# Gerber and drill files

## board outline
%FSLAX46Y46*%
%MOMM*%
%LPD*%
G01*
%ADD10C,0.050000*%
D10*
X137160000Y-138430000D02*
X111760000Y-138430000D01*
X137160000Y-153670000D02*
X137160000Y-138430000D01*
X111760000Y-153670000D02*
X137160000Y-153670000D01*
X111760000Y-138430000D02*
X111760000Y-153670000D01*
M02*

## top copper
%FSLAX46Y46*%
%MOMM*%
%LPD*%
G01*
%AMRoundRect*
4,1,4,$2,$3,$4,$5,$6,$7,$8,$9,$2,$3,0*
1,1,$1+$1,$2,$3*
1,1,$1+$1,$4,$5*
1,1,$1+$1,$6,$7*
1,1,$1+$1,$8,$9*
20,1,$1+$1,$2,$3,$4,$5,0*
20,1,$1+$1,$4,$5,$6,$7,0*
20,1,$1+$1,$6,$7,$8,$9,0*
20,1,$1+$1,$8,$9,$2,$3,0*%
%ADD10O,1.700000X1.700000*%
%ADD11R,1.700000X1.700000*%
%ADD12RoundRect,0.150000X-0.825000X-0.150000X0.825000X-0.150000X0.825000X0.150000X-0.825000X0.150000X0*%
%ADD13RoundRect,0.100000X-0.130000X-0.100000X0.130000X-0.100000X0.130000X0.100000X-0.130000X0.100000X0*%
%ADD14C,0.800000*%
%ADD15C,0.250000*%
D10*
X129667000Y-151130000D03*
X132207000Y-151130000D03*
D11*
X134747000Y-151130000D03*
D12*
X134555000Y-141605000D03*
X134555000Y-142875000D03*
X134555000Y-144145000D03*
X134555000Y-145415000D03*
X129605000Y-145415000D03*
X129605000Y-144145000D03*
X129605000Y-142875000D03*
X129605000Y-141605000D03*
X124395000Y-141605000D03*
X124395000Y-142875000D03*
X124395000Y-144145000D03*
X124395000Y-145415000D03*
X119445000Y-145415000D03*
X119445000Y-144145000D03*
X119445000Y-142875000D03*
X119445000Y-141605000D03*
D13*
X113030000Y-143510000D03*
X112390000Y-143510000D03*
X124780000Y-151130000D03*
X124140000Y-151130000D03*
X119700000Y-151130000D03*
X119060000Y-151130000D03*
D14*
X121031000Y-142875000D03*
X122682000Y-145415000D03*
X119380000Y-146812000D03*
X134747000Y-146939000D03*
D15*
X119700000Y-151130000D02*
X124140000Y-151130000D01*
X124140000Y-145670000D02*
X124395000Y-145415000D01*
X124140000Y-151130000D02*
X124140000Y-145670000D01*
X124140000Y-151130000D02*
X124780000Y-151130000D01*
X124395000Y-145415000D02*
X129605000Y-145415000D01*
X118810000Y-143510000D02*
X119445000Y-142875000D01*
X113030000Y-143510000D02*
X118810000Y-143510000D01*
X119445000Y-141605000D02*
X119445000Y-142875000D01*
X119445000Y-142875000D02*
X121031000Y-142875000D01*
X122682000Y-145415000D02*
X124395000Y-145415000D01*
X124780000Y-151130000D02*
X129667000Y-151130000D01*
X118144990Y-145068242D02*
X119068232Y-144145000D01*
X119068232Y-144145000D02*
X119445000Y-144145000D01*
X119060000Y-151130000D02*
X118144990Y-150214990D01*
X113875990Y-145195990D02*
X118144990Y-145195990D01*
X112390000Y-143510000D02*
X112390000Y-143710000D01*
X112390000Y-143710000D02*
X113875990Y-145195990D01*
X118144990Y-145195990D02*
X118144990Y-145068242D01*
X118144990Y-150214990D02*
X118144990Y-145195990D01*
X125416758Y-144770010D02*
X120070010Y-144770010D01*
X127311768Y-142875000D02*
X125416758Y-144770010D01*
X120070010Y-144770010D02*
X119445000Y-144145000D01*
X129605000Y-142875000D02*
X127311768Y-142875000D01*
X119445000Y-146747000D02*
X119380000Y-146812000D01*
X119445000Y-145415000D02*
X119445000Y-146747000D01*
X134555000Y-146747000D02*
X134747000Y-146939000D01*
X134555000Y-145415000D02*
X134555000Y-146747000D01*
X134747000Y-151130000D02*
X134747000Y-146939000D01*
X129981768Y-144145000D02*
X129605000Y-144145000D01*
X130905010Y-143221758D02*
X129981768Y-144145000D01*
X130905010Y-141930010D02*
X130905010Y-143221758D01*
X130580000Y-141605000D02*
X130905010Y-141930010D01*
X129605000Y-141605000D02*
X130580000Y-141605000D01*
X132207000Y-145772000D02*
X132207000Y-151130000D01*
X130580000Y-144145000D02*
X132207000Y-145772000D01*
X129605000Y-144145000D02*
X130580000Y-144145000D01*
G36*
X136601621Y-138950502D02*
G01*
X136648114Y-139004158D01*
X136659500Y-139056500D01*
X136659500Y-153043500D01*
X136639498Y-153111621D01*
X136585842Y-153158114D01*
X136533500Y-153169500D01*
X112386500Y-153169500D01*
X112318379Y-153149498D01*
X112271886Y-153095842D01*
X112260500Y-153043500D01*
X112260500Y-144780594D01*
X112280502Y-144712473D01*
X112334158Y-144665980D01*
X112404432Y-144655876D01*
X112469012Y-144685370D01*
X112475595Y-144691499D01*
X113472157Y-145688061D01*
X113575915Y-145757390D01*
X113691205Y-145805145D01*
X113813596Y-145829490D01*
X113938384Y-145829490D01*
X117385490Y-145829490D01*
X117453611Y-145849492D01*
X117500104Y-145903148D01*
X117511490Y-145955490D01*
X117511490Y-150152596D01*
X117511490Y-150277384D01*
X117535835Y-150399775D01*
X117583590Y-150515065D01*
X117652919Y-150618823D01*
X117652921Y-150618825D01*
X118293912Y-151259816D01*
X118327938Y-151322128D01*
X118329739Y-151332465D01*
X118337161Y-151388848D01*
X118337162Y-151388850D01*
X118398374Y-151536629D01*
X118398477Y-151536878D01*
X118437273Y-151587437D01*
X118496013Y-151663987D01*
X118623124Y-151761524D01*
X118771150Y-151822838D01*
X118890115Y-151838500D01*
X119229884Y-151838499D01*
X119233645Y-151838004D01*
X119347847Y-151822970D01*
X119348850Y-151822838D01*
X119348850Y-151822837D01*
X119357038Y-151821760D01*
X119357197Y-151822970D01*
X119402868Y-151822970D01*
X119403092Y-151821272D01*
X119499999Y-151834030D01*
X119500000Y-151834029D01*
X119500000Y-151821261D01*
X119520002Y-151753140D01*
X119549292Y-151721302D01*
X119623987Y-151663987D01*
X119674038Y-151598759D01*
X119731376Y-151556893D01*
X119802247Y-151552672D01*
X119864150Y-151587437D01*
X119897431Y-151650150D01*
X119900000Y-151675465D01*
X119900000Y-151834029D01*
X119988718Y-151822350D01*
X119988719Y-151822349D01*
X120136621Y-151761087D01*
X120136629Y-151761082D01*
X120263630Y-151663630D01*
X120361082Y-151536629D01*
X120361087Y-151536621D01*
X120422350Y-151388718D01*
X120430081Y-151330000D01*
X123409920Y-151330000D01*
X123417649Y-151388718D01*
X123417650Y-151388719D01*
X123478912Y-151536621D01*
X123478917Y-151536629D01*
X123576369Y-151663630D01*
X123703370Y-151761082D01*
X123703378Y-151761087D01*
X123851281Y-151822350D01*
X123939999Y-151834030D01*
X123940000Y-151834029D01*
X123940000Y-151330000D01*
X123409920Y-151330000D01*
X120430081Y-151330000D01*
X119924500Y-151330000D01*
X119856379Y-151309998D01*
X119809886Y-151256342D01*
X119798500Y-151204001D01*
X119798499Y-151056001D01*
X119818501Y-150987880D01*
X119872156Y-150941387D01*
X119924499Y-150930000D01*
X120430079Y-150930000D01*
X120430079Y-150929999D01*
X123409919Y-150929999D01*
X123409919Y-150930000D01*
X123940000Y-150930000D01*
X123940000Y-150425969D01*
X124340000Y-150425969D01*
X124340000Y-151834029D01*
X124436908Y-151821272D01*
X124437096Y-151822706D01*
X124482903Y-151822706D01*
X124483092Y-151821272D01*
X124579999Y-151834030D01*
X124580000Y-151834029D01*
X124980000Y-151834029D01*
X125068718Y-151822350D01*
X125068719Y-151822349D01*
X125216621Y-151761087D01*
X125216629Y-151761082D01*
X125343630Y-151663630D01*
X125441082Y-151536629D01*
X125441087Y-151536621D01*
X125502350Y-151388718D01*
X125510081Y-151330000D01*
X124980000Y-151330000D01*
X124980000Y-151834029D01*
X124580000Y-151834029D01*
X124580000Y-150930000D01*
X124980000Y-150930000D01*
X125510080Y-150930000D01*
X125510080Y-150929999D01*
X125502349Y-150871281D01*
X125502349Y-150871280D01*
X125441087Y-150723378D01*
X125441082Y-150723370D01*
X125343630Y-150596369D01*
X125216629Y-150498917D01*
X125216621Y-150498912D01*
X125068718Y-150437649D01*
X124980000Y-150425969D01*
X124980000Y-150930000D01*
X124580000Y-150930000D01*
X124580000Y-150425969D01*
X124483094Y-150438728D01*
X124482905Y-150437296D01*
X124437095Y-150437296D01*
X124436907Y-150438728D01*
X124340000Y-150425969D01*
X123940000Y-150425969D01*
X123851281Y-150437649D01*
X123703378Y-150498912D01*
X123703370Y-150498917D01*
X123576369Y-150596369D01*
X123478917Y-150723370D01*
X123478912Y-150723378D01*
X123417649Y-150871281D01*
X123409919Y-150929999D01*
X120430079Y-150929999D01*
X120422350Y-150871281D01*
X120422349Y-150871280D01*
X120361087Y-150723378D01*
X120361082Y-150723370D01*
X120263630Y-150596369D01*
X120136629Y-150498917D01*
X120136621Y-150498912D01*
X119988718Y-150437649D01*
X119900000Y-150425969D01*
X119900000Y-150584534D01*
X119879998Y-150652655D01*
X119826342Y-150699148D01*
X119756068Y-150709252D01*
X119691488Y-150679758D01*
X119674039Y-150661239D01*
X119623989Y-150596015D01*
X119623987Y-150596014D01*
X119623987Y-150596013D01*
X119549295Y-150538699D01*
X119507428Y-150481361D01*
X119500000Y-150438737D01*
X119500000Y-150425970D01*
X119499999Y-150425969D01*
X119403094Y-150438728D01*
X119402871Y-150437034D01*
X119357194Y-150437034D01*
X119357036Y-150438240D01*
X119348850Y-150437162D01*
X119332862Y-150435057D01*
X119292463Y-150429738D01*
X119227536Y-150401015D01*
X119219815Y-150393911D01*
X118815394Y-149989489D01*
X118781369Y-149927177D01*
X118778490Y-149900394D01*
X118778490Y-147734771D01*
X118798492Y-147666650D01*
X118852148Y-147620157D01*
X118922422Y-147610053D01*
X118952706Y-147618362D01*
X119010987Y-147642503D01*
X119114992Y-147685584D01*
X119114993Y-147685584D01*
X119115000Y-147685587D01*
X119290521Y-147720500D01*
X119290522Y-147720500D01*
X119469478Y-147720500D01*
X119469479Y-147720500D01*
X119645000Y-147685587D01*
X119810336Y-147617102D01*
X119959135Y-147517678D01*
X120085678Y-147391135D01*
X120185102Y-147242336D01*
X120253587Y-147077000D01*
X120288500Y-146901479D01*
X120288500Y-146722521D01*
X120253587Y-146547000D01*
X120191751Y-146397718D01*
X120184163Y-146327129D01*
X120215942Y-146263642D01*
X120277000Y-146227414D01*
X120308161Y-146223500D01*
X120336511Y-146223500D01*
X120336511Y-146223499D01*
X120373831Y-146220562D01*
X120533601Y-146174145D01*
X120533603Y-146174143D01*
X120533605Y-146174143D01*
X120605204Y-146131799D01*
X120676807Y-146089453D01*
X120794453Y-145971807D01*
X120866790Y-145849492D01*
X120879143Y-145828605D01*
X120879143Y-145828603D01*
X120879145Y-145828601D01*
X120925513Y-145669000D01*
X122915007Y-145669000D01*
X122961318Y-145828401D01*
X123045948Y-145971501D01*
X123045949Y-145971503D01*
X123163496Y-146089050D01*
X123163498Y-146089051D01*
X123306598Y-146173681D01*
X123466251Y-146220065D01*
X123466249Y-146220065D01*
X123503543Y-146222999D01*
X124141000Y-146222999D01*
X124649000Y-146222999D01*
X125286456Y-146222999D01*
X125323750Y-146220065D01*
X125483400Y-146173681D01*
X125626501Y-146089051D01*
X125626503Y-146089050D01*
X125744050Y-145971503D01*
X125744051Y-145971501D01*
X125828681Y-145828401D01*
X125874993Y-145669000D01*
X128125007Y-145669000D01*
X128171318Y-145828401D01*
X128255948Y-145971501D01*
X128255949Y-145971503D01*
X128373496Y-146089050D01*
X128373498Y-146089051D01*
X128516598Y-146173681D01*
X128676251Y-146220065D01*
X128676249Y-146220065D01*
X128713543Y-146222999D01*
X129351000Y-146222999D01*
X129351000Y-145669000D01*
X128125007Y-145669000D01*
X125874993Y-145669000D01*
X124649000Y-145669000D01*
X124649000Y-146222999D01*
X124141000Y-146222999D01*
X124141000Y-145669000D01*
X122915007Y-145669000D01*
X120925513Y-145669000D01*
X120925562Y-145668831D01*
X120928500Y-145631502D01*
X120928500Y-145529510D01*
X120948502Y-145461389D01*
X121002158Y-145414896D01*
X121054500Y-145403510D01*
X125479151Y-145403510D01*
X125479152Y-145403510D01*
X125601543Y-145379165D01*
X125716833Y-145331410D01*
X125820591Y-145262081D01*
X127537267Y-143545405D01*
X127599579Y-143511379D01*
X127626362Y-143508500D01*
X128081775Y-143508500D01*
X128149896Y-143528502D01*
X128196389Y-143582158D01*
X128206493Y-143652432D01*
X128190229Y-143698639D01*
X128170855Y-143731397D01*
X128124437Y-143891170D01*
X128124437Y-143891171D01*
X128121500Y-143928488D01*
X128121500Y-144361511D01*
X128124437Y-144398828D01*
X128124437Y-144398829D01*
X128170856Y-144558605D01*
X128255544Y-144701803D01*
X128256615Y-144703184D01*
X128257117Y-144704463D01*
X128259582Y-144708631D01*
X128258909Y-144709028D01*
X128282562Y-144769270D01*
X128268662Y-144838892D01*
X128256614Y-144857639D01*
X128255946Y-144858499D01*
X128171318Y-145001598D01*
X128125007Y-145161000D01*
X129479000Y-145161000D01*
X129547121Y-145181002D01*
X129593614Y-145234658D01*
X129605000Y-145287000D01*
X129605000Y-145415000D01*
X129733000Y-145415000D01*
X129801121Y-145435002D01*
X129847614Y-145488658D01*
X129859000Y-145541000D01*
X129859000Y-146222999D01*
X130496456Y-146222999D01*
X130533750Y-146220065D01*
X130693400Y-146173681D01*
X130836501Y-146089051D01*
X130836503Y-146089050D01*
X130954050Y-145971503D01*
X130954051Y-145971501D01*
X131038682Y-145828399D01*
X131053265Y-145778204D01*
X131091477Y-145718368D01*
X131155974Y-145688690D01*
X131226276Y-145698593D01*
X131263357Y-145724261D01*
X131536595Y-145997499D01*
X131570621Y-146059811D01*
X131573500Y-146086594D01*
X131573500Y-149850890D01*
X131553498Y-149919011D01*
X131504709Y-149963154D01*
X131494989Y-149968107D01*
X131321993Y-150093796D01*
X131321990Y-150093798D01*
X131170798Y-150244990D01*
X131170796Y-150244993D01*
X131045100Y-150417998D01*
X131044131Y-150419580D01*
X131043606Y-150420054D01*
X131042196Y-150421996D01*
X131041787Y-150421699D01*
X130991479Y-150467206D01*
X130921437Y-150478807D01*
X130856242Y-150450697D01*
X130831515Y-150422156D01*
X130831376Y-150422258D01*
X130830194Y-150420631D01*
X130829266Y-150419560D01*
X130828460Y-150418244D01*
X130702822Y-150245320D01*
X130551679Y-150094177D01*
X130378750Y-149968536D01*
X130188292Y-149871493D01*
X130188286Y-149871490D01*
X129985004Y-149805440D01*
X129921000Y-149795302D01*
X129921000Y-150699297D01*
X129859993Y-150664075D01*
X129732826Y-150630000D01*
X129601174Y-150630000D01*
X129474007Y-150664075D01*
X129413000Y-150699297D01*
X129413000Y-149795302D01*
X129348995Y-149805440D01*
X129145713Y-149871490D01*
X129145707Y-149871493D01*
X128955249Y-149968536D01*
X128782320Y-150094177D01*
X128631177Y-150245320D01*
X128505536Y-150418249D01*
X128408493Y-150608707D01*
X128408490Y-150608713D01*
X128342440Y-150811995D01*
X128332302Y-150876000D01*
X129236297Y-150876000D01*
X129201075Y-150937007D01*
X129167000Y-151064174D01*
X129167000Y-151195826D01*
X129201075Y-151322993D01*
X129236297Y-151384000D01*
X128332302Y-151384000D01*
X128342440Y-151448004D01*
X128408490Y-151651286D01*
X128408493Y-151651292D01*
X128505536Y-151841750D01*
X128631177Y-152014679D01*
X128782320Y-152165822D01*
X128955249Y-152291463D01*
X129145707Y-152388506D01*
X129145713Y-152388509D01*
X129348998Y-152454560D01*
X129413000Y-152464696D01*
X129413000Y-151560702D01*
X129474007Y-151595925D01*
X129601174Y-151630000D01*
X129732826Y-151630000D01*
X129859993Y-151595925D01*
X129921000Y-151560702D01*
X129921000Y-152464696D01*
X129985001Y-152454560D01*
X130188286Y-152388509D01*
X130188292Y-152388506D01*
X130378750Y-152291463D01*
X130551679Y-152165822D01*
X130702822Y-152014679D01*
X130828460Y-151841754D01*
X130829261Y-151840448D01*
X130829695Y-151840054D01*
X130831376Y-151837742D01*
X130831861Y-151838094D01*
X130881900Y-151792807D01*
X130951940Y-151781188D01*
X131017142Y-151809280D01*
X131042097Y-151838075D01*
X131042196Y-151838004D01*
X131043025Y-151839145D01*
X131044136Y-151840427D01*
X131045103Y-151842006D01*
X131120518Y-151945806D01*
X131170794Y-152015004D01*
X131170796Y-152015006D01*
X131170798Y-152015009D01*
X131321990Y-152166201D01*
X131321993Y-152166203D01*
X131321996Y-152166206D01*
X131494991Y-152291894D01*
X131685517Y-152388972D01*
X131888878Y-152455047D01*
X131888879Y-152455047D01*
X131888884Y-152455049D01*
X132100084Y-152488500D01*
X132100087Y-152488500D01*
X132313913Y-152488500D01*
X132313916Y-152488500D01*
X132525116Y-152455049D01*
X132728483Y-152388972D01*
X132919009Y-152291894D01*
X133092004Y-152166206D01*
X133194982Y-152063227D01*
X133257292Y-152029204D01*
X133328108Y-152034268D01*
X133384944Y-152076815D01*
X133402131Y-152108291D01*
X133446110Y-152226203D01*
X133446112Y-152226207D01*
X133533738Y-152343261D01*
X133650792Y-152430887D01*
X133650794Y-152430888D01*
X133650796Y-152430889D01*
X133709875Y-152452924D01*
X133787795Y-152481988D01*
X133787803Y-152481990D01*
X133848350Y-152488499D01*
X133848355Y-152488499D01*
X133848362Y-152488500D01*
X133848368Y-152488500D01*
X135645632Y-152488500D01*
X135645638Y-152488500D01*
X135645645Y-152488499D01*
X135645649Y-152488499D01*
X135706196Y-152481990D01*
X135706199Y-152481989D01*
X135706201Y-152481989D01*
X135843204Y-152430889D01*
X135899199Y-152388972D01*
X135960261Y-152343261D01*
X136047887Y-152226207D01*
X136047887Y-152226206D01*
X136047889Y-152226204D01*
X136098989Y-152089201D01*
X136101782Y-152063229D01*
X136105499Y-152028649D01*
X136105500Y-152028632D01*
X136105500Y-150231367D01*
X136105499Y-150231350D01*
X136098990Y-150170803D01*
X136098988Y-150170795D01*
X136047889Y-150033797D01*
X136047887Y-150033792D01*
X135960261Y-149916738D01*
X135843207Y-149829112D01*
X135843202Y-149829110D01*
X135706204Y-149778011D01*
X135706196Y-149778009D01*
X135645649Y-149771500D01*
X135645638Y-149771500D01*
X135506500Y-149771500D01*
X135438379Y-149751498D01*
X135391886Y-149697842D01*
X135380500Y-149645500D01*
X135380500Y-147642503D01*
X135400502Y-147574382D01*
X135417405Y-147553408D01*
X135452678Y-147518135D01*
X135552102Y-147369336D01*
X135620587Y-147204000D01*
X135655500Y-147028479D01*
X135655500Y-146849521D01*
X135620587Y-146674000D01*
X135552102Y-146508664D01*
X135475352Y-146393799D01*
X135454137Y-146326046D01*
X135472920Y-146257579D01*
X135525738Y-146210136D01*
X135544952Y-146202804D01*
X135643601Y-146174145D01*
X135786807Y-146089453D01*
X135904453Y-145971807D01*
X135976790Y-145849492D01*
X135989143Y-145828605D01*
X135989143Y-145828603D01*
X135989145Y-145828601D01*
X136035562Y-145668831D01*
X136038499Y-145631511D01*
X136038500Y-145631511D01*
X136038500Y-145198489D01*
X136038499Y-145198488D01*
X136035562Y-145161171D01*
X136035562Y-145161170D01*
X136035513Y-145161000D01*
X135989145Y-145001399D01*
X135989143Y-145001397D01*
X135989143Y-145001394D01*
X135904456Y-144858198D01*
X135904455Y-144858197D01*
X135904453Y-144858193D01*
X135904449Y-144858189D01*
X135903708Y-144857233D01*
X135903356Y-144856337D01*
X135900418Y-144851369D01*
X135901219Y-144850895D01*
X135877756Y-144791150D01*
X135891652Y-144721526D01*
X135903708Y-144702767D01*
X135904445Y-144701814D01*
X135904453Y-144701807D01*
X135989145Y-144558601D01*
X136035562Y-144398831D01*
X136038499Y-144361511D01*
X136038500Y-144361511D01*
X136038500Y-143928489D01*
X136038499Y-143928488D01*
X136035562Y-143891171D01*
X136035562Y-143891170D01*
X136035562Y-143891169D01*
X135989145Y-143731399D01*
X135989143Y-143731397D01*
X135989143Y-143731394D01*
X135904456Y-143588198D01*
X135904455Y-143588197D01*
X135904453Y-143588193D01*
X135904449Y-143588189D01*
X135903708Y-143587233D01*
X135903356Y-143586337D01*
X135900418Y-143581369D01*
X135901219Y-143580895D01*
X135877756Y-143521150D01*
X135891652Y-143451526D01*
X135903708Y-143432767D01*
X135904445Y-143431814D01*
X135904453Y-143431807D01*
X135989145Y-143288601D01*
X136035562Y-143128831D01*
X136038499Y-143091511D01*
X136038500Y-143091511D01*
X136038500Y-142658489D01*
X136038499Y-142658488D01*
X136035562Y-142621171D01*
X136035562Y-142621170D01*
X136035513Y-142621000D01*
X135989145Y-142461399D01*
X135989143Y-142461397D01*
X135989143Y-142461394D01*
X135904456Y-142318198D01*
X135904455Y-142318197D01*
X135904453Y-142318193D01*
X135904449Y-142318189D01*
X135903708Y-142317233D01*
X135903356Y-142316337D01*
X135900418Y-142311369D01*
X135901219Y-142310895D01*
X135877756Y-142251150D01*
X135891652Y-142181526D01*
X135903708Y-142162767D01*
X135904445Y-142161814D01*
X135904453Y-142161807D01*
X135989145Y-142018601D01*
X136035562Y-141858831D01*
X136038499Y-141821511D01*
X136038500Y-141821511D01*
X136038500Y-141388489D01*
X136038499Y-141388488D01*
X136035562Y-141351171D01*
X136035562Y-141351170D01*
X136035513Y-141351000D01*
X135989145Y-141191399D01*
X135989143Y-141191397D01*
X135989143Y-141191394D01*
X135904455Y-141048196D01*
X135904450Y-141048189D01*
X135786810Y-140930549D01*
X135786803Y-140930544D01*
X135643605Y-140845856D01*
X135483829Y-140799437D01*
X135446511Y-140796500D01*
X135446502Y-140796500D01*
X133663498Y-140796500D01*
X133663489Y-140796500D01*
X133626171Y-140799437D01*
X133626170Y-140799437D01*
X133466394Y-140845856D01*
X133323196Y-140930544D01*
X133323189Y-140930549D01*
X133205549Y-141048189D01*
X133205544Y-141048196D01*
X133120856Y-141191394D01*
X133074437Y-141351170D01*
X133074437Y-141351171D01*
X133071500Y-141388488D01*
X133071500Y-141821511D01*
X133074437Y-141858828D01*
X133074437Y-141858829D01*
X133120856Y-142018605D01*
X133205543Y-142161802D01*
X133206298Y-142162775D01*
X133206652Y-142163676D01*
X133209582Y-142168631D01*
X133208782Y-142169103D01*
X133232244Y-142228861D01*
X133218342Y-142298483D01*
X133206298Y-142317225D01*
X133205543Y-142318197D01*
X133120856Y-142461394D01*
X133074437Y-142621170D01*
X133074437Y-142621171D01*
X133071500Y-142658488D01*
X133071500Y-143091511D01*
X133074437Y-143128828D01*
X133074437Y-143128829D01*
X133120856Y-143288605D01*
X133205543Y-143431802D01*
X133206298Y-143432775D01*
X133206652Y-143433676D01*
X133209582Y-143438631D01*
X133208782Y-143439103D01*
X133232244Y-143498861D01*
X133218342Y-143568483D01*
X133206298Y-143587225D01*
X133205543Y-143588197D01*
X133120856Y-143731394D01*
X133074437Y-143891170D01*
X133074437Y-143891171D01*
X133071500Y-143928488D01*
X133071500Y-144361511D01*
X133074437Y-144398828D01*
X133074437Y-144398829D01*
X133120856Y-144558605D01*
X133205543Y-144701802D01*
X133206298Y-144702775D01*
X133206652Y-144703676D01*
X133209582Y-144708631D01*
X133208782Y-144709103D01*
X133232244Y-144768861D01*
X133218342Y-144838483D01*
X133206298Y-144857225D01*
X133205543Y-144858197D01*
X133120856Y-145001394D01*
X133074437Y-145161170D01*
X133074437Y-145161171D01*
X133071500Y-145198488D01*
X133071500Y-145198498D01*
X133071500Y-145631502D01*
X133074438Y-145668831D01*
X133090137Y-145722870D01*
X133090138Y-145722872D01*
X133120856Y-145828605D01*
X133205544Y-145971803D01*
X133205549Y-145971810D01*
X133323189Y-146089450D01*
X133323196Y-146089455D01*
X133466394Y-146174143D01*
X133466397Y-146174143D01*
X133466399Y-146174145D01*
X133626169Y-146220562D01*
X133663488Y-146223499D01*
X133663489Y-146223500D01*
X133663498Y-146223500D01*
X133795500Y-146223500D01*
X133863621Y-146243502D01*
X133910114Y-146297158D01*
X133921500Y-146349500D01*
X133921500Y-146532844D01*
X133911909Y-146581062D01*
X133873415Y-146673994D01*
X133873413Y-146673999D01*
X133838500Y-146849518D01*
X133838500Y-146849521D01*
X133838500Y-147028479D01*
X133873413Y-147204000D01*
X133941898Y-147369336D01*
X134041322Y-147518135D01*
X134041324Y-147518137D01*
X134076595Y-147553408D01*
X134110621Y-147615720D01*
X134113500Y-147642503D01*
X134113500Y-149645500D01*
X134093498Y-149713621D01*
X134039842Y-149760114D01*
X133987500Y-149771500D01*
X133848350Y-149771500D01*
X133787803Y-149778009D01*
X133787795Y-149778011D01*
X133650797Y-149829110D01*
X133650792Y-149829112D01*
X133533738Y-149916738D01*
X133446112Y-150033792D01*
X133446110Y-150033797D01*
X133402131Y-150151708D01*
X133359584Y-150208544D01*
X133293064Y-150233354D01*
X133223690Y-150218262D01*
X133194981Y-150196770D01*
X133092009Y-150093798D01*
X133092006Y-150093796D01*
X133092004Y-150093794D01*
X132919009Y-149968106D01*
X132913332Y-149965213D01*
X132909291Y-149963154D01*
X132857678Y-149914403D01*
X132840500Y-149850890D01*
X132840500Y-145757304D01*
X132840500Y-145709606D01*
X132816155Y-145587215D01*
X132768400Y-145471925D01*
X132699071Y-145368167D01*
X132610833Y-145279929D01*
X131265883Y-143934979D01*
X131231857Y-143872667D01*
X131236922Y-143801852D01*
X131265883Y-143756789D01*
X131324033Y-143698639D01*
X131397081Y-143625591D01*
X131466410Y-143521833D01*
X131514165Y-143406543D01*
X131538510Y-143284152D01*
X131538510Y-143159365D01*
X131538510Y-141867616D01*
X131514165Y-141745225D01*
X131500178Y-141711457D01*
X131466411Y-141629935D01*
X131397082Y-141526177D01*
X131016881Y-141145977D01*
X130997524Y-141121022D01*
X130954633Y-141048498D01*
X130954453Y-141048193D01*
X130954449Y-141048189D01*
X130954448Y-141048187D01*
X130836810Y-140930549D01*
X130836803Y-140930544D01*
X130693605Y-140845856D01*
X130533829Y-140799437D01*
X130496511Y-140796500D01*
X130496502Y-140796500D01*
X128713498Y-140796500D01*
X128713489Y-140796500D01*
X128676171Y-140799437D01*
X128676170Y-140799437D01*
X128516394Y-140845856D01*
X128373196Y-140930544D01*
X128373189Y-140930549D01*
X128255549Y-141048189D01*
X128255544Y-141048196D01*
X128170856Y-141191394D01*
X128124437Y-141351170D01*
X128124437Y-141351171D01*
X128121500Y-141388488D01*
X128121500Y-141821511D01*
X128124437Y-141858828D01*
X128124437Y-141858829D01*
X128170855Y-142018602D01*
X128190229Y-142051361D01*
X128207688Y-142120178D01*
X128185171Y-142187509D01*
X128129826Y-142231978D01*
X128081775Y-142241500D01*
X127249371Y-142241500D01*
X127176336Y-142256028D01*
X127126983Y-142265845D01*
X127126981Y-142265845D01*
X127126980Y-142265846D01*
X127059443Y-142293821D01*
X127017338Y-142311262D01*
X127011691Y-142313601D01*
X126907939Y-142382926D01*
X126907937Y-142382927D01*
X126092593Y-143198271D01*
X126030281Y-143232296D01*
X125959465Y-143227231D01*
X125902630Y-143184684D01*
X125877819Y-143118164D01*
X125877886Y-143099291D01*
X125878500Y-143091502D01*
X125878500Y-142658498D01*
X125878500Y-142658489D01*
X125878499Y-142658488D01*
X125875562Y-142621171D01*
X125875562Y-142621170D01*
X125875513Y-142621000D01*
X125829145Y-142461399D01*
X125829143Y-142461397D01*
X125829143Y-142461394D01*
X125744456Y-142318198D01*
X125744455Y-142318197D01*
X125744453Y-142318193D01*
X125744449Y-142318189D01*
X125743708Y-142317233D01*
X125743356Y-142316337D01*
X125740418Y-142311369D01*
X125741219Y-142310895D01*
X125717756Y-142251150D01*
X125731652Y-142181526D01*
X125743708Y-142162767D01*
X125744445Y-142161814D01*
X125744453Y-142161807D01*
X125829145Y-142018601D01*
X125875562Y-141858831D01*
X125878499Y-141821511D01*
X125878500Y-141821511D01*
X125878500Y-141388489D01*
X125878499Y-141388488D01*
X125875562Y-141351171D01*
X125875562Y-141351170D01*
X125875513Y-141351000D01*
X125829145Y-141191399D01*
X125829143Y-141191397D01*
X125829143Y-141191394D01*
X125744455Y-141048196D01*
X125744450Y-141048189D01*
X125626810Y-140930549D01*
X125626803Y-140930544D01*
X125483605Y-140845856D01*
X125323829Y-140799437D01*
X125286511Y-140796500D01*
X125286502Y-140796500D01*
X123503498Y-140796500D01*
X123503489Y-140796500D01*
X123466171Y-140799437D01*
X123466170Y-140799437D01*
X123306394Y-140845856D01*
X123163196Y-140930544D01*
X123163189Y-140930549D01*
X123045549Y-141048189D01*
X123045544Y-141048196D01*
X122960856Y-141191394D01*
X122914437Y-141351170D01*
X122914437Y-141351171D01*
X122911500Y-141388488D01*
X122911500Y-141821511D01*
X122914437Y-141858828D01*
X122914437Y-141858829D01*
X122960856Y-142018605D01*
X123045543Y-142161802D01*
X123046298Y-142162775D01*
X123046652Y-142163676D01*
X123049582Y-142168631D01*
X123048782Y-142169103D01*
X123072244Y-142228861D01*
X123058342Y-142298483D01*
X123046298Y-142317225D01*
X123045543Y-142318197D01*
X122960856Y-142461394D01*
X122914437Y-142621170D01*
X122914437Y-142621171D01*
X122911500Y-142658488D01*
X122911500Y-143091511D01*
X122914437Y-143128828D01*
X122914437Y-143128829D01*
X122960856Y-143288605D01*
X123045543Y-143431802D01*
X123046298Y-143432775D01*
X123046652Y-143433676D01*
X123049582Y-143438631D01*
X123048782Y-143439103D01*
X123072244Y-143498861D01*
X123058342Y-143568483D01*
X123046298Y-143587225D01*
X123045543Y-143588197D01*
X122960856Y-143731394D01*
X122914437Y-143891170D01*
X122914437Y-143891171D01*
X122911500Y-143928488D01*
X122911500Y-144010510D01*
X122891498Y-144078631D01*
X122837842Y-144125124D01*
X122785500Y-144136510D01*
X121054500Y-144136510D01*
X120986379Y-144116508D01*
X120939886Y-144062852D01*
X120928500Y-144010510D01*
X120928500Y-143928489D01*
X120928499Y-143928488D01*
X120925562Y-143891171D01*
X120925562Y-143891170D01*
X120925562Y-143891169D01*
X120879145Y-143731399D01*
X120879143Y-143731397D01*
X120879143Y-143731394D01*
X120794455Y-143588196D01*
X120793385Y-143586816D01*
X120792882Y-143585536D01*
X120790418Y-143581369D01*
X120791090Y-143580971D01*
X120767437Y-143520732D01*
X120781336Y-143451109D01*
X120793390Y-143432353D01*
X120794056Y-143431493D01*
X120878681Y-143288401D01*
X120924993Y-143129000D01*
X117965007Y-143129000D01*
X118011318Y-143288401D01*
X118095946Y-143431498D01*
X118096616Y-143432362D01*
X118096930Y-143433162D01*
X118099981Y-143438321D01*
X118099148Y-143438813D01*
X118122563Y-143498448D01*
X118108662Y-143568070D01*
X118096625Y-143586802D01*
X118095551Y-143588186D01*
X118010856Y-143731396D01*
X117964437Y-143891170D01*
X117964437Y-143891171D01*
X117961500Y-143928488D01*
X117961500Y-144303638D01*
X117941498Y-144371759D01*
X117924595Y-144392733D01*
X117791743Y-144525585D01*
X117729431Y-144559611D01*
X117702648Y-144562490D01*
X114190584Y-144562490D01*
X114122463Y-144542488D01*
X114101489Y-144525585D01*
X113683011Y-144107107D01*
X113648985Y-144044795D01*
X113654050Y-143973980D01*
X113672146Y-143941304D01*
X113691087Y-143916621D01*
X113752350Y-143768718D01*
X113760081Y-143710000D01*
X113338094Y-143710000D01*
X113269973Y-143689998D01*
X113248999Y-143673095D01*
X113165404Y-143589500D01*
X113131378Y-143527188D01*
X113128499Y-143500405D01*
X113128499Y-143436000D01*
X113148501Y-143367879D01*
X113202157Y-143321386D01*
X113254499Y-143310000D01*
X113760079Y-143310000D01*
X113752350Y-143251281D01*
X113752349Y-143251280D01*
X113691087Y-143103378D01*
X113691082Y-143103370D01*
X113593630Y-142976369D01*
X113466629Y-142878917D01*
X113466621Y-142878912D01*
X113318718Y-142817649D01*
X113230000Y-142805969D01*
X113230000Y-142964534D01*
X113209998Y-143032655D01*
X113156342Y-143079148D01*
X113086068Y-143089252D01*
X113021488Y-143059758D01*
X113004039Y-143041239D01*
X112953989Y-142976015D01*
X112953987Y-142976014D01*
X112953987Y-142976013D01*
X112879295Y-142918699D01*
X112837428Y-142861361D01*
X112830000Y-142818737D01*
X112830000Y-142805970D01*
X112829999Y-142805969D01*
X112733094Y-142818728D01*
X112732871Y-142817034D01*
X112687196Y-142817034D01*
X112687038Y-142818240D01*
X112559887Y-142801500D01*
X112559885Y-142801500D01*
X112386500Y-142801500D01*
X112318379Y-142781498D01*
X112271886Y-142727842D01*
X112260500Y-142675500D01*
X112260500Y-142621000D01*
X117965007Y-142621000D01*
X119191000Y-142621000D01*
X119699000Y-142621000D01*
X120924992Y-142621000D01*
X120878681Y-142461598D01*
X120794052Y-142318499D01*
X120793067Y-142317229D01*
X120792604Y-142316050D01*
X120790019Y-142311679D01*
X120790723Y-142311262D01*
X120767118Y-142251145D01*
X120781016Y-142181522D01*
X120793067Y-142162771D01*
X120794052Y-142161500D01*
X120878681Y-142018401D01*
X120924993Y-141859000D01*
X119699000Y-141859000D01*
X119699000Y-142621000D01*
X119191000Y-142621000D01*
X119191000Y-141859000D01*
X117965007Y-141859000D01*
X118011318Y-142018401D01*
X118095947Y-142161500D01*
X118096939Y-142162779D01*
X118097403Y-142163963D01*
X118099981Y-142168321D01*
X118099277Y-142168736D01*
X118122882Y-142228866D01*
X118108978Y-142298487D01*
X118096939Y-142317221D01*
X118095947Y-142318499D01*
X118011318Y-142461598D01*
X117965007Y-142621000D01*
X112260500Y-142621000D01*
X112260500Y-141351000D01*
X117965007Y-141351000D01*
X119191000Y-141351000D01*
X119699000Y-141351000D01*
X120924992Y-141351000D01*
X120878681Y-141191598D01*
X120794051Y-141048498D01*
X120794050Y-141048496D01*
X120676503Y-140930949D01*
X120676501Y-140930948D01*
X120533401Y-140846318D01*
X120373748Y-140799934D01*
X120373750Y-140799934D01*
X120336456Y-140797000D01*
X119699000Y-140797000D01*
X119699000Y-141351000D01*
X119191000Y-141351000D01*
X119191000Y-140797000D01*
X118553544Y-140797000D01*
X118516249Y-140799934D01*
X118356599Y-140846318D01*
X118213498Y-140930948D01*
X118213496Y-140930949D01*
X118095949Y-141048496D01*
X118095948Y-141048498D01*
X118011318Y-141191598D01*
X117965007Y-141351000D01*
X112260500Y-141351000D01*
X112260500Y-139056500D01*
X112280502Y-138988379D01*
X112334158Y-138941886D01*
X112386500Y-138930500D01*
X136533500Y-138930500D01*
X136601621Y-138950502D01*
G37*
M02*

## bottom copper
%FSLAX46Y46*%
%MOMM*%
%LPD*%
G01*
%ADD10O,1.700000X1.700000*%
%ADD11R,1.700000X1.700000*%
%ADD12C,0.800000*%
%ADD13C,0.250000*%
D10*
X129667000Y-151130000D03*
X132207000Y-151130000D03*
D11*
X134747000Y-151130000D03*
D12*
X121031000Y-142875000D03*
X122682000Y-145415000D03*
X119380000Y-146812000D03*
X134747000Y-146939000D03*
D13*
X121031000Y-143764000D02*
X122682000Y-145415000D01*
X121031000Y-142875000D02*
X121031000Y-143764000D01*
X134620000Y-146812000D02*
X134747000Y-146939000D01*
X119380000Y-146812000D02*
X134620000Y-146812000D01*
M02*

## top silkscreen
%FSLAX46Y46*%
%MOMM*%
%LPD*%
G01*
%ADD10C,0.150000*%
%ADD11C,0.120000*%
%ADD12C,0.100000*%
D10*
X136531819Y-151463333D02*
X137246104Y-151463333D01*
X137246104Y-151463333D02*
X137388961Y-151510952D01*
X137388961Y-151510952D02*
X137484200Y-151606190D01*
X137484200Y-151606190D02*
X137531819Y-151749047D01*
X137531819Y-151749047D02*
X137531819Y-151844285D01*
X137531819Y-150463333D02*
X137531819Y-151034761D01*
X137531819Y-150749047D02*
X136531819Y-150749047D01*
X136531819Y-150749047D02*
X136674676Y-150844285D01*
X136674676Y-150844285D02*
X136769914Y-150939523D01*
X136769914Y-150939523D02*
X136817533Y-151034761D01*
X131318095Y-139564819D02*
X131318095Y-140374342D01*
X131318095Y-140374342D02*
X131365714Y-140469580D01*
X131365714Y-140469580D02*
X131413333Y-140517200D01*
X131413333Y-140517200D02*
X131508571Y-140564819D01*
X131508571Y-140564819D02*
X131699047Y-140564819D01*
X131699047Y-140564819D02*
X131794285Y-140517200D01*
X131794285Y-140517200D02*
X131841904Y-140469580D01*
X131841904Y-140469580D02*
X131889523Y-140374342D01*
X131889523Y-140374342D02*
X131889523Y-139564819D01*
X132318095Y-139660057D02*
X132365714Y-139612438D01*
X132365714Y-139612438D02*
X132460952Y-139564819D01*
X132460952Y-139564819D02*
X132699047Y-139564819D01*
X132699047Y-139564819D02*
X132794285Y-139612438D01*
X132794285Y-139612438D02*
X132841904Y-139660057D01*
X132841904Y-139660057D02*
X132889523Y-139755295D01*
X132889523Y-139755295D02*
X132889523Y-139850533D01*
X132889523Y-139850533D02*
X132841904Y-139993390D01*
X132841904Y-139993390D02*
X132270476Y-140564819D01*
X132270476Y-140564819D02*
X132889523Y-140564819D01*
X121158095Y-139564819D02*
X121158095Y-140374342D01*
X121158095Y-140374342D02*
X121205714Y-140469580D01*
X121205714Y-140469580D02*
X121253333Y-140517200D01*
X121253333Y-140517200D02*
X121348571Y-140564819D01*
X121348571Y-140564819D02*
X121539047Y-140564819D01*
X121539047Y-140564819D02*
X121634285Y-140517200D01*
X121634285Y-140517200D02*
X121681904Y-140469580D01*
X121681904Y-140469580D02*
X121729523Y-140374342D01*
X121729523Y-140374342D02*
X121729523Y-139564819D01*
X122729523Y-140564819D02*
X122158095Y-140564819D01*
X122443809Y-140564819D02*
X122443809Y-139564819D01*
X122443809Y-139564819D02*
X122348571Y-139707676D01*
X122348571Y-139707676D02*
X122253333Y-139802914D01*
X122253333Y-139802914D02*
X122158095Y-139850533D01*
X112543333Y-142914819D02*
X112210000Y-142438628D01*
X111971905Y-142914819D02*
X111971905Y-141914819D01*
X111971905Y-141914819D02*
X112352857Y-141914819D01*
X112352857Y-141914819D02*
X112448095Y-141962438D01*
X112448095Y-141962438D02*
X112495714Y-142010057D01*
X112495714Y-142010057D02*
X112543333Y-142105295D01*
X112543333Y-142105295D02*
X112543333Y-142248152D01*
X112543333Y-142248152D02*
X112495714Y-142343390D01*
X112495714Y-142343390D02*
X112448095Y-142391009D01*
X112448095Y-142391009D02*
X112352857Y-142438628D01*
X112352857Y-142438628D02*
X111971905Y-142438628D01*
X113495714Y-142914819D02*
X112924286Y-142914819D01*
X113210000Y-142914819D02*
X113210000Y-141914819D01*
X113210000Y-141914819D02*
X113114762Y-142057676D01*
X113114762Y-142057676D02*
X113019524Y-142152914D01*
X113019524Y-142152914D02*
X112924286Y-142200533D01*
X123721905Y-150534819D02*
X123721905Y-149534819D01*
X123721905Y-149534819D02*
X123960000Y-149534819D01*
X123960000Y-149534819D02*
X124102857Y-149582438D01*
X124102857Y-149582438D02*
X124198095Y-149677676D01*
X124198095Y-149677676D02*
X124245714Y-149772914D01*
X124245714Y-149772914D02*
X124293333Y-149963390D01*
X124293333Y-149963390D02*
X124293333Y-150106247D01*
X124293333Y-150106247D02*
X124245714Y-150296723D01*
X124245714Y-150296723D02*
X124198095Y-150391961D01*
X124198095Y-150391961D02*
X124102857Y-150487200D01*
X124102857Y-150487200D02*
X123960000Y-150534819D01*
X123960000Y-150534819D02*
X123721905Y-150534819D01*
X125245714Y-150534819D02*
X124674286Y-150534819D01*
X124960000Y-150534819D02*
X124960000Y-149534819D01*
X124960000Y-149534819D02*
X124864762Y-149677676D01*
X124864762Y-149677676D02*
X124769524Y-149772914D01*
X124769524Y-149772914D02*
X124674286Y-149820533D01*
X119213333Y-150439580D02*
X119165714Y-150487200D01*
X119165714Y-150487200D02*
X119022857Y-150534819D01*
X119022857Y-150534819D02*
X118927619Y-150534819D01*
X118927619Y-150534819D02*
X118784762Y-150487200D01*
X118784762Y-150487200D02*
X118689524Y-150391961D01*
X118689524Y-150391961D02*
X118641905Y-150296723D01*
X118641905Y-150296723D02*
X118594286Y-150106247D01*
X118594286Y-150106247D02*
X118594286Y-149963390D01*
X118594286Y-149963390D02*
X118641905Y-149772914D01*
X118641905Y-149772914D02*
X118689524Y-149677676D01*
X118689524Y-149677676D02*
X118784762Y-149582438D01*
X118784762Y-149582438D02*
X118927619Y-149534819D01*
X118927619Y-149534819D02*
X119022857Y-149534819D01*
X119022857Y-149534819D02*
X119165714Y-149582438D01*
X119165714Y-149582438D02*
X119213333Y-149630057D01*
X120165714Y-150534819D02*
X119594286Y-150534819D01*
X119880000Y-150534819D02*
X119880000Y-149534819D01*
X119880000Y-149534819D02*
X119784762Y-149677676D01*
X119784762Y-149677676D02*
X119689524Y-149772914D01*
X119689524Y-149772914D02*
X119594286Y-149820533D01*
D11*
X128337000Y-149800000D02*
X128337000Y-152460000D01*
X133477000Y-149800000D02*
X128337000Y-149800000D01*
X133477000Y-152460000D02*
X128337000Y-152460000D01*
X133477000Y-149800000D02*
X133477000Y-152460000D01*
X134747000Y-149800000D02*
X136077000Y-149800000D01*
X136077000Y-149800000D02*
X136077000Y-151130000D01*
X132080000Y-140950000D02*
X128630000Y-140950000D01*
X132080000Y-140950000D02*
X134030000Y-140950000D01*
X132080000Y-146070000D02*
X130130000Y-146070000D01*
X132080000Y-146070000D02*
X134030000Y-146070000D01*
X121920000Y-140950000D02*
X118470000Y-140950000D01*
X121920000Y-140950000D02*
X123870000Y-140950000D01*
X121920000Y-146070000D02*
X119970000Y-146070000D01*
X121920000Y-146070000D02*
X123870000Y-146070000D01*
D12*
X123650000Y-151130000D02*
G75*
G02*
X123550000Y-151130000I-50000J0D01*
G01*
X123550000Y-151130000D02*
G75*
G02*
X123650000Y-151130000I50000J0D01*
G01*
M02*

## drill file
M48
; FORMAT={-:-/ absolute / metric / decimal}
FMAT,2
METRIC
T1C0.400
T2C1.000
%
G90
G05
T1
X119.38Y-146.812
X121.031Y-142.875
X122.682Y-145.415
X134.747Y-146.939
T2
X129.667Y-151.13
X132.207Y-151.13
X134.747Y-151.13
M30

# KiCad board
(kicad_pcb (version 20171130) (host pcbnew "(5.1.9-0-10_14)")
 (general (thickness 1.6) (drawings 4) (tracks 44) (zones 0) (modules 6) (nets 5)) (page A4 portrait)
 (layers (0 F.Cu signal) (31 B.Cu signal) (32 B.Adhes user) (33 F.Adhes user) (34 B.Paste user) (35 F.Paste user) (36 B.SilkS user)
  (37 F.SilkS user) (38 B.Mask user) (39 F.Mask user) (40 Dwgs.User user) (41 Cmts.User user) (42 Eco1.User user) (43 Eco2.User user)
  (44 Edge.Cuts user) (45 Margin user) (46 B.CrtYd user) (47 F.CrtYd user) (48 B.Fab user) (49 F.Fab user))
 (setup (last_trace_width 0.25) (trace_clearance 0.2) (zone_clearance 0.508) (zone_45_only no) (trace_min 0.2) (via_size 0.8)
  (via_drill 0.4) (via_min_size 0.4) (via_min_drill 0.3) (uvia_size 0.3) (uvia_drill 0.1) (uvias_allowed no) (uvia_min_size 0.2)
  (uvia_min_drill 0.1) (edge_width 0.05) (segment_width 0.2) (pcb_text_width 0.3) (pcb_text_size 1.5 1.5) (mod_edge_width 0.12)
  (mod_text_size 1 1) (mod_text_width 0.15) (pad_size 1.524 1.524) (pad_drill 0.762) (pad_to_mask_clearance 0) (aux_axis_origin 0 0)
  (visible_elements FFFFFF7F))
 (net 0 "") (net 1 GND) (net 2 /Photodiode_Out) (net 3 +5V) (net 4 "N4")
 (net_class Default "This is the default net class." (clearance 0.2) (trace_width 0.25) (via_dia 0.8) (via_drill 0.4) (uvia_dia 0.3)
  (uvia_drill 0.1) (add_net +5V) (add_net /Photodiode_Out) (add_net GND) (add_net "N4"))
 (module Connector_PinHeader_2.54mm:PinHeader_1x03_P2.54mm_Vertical (layer F.Cu) (at 134.747 151.13 270)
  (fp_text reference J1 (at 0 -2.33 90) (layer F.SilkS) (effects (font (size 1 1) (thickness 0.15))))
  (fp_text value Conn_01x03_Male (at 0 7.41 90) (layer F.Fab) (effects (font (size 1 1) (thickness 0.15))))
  (fp_line (start -1.33 6.41) (end 1.33 6.41) (layer F.SilkS) (width 0.12))
  (fp_line (start -1.33 1.27) (end -1.33 6.41) (layer F.SilkS) (width 0.12))
  (fp_line (start 1.33 1.27) (end 1.33 6.41) (layer F.SilkS) (width 0.12))
  (fp_line (start -1.33 1.27) (end 1.33 1.27) (layer F.SilkS) (width 0.12))
  (fp_line (start -1.33 0) (end -1.33 -1.33) (layer F.SilkS) (width 0.12))
  (fp_line (start -1.33 -1.33) (end 0 -1.33) (layer F.SilkS) (width 0.12))
  (pad 3 thru_hole oval (at 0 5.08 270) (size 1.7 1.7) (drill 1) (layers *.Cu *.Mask) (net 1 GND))
  (pad 2 thru_hole oval (at 0 2.54 270) (size 1.7 1.7) (drill 1) (layers *.Cu *.Mask) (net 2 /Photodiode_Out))
  (pad 1 thru_hole rect (at 0 0 270) (size 1.7 1.7) (drill 1) (layers *.Cu *.Mask) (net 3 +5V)))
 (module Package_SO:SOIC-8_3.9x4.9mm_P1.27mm (layer F.Cu) (at 132.08 143.51)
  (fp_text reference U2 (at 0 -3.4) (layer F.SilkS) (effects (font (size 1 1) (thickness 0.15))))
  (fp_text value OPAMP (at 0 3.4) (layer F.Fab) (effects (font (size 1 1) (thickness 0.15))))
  (fp_line (start 0 -2.56) (end -3.45 -2.56) (layer F.SilkS) (width 0.12))
  (fp_line (start 0 -2.56) (end 1.95 -2.56) (layer F.SilkS) (width 0.12))
  (fp_line (start 0 2.56) (end -1.95 2.56) (layer F.SilkS) (width 0.12))
  (fp_line (start 0 2.56) (end 1.95 2.56) (layer F.SilkS) (width 0.12))
  (pad 8 smd roundrect (at 2.475 -1.905) (size 1.95 0.6) (layers F.Cu F.Paste F.Mask) (roundrect_rratio 0.25))
  (pad 7 smd roundrect (at 2.475 -0.635) (size 1.95 0.6) (layers F.Cu F.Paste F.Mask) (roundrect_rratio 0.25))
  (pad 6 smd roundrect (at 2.475 0.635) (size 1.95 0.6) (layers F.Cu F.Paste F.Mask) (roundrect_rratio 0.25))
  (pad 5 smd roundrect (at 2.475 1.905) (size 1.95 0.6) (layers F.Cu F.Paste F.Mask) (roundrect_rratio 0.25) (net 3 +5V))
  (pad 4 smd roundrect (at -2.475 1.905) (size 1.95 0.6) (layers F.Cu F.Paste F.Mask) (roundrect_rratio 0.25) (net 1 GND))
  (pad 3 smd roundrect (at -2.475 0.635) (size 1.95 0.6) (layers F.Cu F.Paste F.Mask) (roundrect_rratio 0.25) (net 2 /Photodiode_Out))
  (pad 2 smd roundrect (at -2.475 -0.635) (size 1.95 0.6) (layers F.Cu F.Paste F.Mask) (roundrect_rratio 0.25) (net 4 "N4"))
  (pad 1 smd roundrect (at -2.475 -1.905) (size 1.95 0.6) (layers F.Cu F.Paste F.Mask) (roundrect_rratio 0.25) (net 2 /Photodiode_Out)))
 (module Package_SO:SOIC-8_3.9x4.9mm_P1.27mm (layer F.Cu) (at 121.92 143.51)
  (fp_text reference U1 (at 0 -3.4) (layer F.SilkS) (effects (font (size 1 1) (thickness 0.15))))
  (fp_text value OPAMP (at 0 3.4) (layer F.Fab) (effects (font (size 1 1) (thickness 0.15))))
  (fp_line (start 0 -2.56) (end -3.45 -2.56) (layer F.SilkS) (width 0.12))
  (fp_line (start 0 -2.56) (end 1.95 -2.56) (layer F.SilkS) (width 0.12))
  (fp_line (start 0 2.56) (end -1.95 2.56) (layer F.SilkS) (width 0.12))
  (fp_line (start 0 2.56) (end 1.95 2.56) (layer F.SilkS) (width 0.12))
  (pad 8 smd roundrect (at 2.475 -1.905) (size 1.95 0.6) (layers F.Cu F.Paste F.Mask) (roundrect_rratio 0.25))
  (pad 7 smd roundrect (at 2.475 -0.635) (size 1.95 0.6) (layers F.Cu F.Paste F.Mask) (roundrect_rratio 0.25))
  (pad 6 smd roundrect (at 2.475 0.635) (size 1.95 0.6) (layers F.Cu F.Paste F.Mask) (roundrect_rratio 0.25))
  (pad 5 smd roundrect (at 2.475 1.905) (size 1.95 0.6) (layers F.Cu F.Paste F.Mask) (roundrect_rratio 0.25) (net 1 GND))
  (pad 4 smd roundrect (at -2.475 1.905) (size 1.95 0.6) (layers F.Cu F.Paste F.Mask) (roundrect_rratio 0.25) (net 3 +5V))
  (pad 3 smd roundrect (at -2.475 0.635) (size 1.95 0.6) (layers F.Cu F.Paste F.Mask) (roundrect_rratio 0.25) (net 4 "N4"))
  (pad 2 smd roundrect (at -2.475 -0.635) (size 1.95 0.6) (layers F.Cu F.Paste F.Mask) (roundrect_rratio 0.25) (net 1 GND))
  (pad 1 smd roundrect (at -2.475 -1.905) (size 1.95 0.6) (layers F.Cu F.Paste F.Mask) (roundrect_rratio 0.25) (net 1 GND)))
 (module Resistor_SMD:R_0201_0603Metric (layer F.Cu) (at 112.71 143.51)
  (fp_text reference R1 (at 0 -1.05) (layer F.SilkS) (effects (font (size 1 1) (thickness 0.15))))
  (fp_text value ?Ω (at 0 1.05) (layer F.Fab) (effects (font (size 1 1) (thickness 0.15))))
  (pad 2 smd roundrect (at 0.32 0) (size 0.46 0.4) (layers F.Cu F.Mask) (roundrect_rratio 0.25) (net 1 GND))
  (pad 1 smd roundrect (at -0.32 0) (size 0.46 0.4) (layers F.Cu F.Mask) (roundrect_rratio 0.25) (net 4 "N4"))
  (pad "" smd roundrect (at 0.345 0) (size 0.318 0.36) (layers F.Paste) (roundrect_rratio 0.25))
  (pad "" smd roundrect (at -0.345 0) (size 0.318 0.36) (layers F.Paste) (roundrect_rratio 0.25)))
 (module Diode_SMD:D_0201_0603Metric (layer F.Cu) (at 124.46 151.13)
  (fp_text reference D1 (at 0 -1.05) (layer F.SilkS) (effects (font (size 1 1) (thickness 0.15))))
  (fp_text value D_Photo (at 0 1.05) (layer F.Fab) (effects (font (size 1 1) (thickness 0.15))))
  (fp_circle (center -0.86 0) (end -0.81 0) (layer F.SilkS) (width 0.1))
  (pad 2 smd roundrect (at 0.32 0) (size 0.46 0.4) (layers F.Cu F.Mask) (roundrect_rratio 0.25) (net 1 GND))
  (pad 1 smd roundrect (at -0.32 0) (size 0.46 0.4) (layers F.Cu F.Mask) (roundrect_rratio 0.25) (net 1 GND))
  (pad "" smd roundrect (at 0.345 0) (size 0.318 0.36) (layers F.Paste) (roundrect_rratio 0.25))
  (pad "" smd roundrect (at -0.345 0) (size 0.318 0.36) (layers F.Paste) (roundrect_rratio 0.25)))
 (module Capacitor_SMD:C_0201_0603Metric (layer F.Cu) (at 119.38 151.13)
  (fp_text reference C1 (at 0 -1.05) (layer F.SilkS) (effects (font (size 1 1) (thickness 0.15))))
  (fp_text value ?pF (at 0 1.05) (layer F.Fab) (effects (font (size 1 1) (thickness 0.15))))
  (pad 2 smd roundrect (at 0.32 0) (size 0.46 0.4) (layers F.Cu F.Mask) (roundrect_rratio 0.25) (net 1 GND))
  (pad 1 smd roundrect (at -0.32 0) (size 0.46 0.4) (layers F.Cu F.Mask) (roundrect_rratio 0.25) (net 4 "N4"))
  (pad "" smd roundrect (at 0.345 0) (size 0.318 0.36) (layers F.Paste) (roundrect_rratio 0.25))
  (pad "" smd roundrect (at -0.345 0) (size 0.318 0.36) (layers F.Paste) (roundrect_rratio 0.25)))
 (gr_line (start 137.16 138.43) (end 111.76 138.43) (layer Edge.Cuts) (width 0.05))
 (gr_line (start 137.16 153.67) (end 137.16 138.43) (layer Edge.Cuts) (width 0.05))
 (gr_line (start 111.76 153.67) (end 137.16 153.67) (layer Edge.Cuts) (width 0.05))
 (gr_line (start 111.76 138.43) (end 111.76 153.67) (layer Edge.Cuts) (width 0.05))
 (via (at 121.031 142.875) (size 0.8) (drill 0.4) (layers F.Cu B.Cu) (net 1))
 (via (at 122.682 145.415) (size 0.8) (drill 0.4) (layers F.Cu B.Cu) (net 1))
 (via (at 119.38 146.812) (size 0.8) (drill 0.4) (layers F.Cu B.Cu) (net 3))
 (via (at 134.747 146.939) (size 0.8) (drill 0.4) (layers F.Cu B.Cu) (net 3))
 (segment (start 119.7 151.13) (end 124.14 151.13) (width 0.25) (layer F.Cu) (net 1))
 (segment (start 124.14 145.67) (end 124.395 145.415) (width 0.25) (layer F.Cu) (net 1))
 (segment (start 124.14 151.13) (end 124.14 145.67) (width 0.25) (layer F.Cu) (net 1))
 (segment (start 124.14 151.13) (end 124.78 151.13) (width 0.25) (layer F.Cu) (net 1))
 (segment (start 124.395 145.415) (end 129.605 145.415) (width 0.25) (layer F.Cu) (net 1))
 (segment (start 118.81 143.51) (end 119.445 142.875) (width 0.25) (layer F.Cu) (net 1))
 (segment (start 113.03 143.51) (end 118.81 143.51) (width 0.25) (layer F.Cu) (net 1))
 (segment (start 119.445 141.605) (end 119.445 142.875) (width 0.25) (layer F.Cu) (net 1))
 (segment (start 119.445 142.875) (end 121.031 142.875) (width 0.25) (layer F.Cu) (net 1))
 (segment (start 122.682 145.415) (end 124.395 145.415) (width 0.25) (layer F.Cu) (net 1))
 (segment (start 121.031 143.764) (end 122.682 145.415) (width 0.25) (layer B.Cu) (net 1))
 (segment (start 121.031 142.875) (end 121.031 143.764) (width 0.25) (layer B.Cu) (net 1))
 (segment (start 124.78 151.13) (end 129.667 151.13) (width 0.25) (layer F.Cu) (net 1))
 (segment (start 118.14499 145.068242) (end 119.068232 144.145) (width 0.25) (layer F.Cu) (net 4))
 (segment (start 119.068232 144.145) (end 119.445 144.145) (width 0.25) (layer F.Cu) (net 4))
 (segment (start 119.06 151.13) (end 118.14499 150.21499) (width 0.25) (layer F.Cu) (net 4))
 (segment (start 113.87599 145.19599) (end 118.14499 145.19599) (width 0.25) (layer F.Cu) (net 4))
 (segment (start 112.39 143.51) (end 112.39 143.71) (width 0.25) (layer F.Cu) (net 4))
 (segment (start 112.39 143.71) (end 113.87599 145.19599) (width 0.25) (layer F.Cu) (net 4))
 (segment (start 118.14499 145.19599) (end 118.14499 145.068242) (width 0.25) (layer F.Cu) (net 4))
 (segment (start 118.14499 150.21499) (end 118.14499 145.19599) (width 0.25) (layer F.Cu) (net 4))
 (segment (start 125.416758 144.77001) (end 120.07001 144.77001) (width 0.25) (layer F.Cu) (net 4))
 (segment (start 127.311768 142.875) (end 125.416758 144.77001) (width 0.25) (layer F.Cu) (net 4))
 (segment (start 120.07001 144.77001) (end 119.445 144.145) (width 0.25) (layer F.Cu) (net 4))
 (segment (start 129.605 142.875) (end 127.311768 142.875) (width 0.25) (layer F.Cu) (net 4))
 (segment (start 119.445 146.747) (end 119.38 146.812) (width 0.25) (layer F.Cu) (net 3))
 (segment (start 119.445 145.415) (end 119.445 146.747) (width 0.25) (layer F.Cu) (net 3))
 (segment (start 134.555 146.747) (end 134.747 146.939) (width 0.25) (layer F.Cu) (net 3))
 (segment (start 134.555 145.415) (end 134.555 146.747) (width 0.25) (layer F.Cu) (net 3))
 (segment (start 134.62 146.812) (end 134.747 146.939) (width 0.25) (layer B.Cu) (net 3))
 (segment (start 119.38 146.812) (end 134.62 146.812) (width 0.25) (layer B.Cu) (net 3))
 (segment (start 134.747 151.13) (end 134.747 146.939) (width 0.25) (layer F.Cu) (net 3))
 (segment (start 129.981768 144.145) (end 129.605 144.145) (width 0.25) (layer F.Cu) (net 2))
 (segment (start 130.90501 143.221758) (end 129.981768 144.145) (width 0.25) (layer F.Cu) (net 2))
 (segment (start 130.90501 141.93001) (end 130.90501 143.221758) (width 0.25) (layer F.Cu) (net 2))
 (segment (start 130.58 141.605) (end 130.90501 141.93001) (width 0.25) (layer F.Cu) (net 2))
 (segment (start 129.605 141.605) (end 130.58 141.605) (width 0.25) (layer F.Cu) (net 2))
 (segment (start 132.207 145.772) (end 132.207 151.13) (width 0.25) (layer F.Cu) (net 2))
 (segment (start 130.58 144.145) (end 132.207 145.772) (width 0.25) (layer F.Cu) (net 2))
 (segment (start 129.605 144.145) (end 130.58 144.145) (width 0.25) (layer F.Cu) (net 2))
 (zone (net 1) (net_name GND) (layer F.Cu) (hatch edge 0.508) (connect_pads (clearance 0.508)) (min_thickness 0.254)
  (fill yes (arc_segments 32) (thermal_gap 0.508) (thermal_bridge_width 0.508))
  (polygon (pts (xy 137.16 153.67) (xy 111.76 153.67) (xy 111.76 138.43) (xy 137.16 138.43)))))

